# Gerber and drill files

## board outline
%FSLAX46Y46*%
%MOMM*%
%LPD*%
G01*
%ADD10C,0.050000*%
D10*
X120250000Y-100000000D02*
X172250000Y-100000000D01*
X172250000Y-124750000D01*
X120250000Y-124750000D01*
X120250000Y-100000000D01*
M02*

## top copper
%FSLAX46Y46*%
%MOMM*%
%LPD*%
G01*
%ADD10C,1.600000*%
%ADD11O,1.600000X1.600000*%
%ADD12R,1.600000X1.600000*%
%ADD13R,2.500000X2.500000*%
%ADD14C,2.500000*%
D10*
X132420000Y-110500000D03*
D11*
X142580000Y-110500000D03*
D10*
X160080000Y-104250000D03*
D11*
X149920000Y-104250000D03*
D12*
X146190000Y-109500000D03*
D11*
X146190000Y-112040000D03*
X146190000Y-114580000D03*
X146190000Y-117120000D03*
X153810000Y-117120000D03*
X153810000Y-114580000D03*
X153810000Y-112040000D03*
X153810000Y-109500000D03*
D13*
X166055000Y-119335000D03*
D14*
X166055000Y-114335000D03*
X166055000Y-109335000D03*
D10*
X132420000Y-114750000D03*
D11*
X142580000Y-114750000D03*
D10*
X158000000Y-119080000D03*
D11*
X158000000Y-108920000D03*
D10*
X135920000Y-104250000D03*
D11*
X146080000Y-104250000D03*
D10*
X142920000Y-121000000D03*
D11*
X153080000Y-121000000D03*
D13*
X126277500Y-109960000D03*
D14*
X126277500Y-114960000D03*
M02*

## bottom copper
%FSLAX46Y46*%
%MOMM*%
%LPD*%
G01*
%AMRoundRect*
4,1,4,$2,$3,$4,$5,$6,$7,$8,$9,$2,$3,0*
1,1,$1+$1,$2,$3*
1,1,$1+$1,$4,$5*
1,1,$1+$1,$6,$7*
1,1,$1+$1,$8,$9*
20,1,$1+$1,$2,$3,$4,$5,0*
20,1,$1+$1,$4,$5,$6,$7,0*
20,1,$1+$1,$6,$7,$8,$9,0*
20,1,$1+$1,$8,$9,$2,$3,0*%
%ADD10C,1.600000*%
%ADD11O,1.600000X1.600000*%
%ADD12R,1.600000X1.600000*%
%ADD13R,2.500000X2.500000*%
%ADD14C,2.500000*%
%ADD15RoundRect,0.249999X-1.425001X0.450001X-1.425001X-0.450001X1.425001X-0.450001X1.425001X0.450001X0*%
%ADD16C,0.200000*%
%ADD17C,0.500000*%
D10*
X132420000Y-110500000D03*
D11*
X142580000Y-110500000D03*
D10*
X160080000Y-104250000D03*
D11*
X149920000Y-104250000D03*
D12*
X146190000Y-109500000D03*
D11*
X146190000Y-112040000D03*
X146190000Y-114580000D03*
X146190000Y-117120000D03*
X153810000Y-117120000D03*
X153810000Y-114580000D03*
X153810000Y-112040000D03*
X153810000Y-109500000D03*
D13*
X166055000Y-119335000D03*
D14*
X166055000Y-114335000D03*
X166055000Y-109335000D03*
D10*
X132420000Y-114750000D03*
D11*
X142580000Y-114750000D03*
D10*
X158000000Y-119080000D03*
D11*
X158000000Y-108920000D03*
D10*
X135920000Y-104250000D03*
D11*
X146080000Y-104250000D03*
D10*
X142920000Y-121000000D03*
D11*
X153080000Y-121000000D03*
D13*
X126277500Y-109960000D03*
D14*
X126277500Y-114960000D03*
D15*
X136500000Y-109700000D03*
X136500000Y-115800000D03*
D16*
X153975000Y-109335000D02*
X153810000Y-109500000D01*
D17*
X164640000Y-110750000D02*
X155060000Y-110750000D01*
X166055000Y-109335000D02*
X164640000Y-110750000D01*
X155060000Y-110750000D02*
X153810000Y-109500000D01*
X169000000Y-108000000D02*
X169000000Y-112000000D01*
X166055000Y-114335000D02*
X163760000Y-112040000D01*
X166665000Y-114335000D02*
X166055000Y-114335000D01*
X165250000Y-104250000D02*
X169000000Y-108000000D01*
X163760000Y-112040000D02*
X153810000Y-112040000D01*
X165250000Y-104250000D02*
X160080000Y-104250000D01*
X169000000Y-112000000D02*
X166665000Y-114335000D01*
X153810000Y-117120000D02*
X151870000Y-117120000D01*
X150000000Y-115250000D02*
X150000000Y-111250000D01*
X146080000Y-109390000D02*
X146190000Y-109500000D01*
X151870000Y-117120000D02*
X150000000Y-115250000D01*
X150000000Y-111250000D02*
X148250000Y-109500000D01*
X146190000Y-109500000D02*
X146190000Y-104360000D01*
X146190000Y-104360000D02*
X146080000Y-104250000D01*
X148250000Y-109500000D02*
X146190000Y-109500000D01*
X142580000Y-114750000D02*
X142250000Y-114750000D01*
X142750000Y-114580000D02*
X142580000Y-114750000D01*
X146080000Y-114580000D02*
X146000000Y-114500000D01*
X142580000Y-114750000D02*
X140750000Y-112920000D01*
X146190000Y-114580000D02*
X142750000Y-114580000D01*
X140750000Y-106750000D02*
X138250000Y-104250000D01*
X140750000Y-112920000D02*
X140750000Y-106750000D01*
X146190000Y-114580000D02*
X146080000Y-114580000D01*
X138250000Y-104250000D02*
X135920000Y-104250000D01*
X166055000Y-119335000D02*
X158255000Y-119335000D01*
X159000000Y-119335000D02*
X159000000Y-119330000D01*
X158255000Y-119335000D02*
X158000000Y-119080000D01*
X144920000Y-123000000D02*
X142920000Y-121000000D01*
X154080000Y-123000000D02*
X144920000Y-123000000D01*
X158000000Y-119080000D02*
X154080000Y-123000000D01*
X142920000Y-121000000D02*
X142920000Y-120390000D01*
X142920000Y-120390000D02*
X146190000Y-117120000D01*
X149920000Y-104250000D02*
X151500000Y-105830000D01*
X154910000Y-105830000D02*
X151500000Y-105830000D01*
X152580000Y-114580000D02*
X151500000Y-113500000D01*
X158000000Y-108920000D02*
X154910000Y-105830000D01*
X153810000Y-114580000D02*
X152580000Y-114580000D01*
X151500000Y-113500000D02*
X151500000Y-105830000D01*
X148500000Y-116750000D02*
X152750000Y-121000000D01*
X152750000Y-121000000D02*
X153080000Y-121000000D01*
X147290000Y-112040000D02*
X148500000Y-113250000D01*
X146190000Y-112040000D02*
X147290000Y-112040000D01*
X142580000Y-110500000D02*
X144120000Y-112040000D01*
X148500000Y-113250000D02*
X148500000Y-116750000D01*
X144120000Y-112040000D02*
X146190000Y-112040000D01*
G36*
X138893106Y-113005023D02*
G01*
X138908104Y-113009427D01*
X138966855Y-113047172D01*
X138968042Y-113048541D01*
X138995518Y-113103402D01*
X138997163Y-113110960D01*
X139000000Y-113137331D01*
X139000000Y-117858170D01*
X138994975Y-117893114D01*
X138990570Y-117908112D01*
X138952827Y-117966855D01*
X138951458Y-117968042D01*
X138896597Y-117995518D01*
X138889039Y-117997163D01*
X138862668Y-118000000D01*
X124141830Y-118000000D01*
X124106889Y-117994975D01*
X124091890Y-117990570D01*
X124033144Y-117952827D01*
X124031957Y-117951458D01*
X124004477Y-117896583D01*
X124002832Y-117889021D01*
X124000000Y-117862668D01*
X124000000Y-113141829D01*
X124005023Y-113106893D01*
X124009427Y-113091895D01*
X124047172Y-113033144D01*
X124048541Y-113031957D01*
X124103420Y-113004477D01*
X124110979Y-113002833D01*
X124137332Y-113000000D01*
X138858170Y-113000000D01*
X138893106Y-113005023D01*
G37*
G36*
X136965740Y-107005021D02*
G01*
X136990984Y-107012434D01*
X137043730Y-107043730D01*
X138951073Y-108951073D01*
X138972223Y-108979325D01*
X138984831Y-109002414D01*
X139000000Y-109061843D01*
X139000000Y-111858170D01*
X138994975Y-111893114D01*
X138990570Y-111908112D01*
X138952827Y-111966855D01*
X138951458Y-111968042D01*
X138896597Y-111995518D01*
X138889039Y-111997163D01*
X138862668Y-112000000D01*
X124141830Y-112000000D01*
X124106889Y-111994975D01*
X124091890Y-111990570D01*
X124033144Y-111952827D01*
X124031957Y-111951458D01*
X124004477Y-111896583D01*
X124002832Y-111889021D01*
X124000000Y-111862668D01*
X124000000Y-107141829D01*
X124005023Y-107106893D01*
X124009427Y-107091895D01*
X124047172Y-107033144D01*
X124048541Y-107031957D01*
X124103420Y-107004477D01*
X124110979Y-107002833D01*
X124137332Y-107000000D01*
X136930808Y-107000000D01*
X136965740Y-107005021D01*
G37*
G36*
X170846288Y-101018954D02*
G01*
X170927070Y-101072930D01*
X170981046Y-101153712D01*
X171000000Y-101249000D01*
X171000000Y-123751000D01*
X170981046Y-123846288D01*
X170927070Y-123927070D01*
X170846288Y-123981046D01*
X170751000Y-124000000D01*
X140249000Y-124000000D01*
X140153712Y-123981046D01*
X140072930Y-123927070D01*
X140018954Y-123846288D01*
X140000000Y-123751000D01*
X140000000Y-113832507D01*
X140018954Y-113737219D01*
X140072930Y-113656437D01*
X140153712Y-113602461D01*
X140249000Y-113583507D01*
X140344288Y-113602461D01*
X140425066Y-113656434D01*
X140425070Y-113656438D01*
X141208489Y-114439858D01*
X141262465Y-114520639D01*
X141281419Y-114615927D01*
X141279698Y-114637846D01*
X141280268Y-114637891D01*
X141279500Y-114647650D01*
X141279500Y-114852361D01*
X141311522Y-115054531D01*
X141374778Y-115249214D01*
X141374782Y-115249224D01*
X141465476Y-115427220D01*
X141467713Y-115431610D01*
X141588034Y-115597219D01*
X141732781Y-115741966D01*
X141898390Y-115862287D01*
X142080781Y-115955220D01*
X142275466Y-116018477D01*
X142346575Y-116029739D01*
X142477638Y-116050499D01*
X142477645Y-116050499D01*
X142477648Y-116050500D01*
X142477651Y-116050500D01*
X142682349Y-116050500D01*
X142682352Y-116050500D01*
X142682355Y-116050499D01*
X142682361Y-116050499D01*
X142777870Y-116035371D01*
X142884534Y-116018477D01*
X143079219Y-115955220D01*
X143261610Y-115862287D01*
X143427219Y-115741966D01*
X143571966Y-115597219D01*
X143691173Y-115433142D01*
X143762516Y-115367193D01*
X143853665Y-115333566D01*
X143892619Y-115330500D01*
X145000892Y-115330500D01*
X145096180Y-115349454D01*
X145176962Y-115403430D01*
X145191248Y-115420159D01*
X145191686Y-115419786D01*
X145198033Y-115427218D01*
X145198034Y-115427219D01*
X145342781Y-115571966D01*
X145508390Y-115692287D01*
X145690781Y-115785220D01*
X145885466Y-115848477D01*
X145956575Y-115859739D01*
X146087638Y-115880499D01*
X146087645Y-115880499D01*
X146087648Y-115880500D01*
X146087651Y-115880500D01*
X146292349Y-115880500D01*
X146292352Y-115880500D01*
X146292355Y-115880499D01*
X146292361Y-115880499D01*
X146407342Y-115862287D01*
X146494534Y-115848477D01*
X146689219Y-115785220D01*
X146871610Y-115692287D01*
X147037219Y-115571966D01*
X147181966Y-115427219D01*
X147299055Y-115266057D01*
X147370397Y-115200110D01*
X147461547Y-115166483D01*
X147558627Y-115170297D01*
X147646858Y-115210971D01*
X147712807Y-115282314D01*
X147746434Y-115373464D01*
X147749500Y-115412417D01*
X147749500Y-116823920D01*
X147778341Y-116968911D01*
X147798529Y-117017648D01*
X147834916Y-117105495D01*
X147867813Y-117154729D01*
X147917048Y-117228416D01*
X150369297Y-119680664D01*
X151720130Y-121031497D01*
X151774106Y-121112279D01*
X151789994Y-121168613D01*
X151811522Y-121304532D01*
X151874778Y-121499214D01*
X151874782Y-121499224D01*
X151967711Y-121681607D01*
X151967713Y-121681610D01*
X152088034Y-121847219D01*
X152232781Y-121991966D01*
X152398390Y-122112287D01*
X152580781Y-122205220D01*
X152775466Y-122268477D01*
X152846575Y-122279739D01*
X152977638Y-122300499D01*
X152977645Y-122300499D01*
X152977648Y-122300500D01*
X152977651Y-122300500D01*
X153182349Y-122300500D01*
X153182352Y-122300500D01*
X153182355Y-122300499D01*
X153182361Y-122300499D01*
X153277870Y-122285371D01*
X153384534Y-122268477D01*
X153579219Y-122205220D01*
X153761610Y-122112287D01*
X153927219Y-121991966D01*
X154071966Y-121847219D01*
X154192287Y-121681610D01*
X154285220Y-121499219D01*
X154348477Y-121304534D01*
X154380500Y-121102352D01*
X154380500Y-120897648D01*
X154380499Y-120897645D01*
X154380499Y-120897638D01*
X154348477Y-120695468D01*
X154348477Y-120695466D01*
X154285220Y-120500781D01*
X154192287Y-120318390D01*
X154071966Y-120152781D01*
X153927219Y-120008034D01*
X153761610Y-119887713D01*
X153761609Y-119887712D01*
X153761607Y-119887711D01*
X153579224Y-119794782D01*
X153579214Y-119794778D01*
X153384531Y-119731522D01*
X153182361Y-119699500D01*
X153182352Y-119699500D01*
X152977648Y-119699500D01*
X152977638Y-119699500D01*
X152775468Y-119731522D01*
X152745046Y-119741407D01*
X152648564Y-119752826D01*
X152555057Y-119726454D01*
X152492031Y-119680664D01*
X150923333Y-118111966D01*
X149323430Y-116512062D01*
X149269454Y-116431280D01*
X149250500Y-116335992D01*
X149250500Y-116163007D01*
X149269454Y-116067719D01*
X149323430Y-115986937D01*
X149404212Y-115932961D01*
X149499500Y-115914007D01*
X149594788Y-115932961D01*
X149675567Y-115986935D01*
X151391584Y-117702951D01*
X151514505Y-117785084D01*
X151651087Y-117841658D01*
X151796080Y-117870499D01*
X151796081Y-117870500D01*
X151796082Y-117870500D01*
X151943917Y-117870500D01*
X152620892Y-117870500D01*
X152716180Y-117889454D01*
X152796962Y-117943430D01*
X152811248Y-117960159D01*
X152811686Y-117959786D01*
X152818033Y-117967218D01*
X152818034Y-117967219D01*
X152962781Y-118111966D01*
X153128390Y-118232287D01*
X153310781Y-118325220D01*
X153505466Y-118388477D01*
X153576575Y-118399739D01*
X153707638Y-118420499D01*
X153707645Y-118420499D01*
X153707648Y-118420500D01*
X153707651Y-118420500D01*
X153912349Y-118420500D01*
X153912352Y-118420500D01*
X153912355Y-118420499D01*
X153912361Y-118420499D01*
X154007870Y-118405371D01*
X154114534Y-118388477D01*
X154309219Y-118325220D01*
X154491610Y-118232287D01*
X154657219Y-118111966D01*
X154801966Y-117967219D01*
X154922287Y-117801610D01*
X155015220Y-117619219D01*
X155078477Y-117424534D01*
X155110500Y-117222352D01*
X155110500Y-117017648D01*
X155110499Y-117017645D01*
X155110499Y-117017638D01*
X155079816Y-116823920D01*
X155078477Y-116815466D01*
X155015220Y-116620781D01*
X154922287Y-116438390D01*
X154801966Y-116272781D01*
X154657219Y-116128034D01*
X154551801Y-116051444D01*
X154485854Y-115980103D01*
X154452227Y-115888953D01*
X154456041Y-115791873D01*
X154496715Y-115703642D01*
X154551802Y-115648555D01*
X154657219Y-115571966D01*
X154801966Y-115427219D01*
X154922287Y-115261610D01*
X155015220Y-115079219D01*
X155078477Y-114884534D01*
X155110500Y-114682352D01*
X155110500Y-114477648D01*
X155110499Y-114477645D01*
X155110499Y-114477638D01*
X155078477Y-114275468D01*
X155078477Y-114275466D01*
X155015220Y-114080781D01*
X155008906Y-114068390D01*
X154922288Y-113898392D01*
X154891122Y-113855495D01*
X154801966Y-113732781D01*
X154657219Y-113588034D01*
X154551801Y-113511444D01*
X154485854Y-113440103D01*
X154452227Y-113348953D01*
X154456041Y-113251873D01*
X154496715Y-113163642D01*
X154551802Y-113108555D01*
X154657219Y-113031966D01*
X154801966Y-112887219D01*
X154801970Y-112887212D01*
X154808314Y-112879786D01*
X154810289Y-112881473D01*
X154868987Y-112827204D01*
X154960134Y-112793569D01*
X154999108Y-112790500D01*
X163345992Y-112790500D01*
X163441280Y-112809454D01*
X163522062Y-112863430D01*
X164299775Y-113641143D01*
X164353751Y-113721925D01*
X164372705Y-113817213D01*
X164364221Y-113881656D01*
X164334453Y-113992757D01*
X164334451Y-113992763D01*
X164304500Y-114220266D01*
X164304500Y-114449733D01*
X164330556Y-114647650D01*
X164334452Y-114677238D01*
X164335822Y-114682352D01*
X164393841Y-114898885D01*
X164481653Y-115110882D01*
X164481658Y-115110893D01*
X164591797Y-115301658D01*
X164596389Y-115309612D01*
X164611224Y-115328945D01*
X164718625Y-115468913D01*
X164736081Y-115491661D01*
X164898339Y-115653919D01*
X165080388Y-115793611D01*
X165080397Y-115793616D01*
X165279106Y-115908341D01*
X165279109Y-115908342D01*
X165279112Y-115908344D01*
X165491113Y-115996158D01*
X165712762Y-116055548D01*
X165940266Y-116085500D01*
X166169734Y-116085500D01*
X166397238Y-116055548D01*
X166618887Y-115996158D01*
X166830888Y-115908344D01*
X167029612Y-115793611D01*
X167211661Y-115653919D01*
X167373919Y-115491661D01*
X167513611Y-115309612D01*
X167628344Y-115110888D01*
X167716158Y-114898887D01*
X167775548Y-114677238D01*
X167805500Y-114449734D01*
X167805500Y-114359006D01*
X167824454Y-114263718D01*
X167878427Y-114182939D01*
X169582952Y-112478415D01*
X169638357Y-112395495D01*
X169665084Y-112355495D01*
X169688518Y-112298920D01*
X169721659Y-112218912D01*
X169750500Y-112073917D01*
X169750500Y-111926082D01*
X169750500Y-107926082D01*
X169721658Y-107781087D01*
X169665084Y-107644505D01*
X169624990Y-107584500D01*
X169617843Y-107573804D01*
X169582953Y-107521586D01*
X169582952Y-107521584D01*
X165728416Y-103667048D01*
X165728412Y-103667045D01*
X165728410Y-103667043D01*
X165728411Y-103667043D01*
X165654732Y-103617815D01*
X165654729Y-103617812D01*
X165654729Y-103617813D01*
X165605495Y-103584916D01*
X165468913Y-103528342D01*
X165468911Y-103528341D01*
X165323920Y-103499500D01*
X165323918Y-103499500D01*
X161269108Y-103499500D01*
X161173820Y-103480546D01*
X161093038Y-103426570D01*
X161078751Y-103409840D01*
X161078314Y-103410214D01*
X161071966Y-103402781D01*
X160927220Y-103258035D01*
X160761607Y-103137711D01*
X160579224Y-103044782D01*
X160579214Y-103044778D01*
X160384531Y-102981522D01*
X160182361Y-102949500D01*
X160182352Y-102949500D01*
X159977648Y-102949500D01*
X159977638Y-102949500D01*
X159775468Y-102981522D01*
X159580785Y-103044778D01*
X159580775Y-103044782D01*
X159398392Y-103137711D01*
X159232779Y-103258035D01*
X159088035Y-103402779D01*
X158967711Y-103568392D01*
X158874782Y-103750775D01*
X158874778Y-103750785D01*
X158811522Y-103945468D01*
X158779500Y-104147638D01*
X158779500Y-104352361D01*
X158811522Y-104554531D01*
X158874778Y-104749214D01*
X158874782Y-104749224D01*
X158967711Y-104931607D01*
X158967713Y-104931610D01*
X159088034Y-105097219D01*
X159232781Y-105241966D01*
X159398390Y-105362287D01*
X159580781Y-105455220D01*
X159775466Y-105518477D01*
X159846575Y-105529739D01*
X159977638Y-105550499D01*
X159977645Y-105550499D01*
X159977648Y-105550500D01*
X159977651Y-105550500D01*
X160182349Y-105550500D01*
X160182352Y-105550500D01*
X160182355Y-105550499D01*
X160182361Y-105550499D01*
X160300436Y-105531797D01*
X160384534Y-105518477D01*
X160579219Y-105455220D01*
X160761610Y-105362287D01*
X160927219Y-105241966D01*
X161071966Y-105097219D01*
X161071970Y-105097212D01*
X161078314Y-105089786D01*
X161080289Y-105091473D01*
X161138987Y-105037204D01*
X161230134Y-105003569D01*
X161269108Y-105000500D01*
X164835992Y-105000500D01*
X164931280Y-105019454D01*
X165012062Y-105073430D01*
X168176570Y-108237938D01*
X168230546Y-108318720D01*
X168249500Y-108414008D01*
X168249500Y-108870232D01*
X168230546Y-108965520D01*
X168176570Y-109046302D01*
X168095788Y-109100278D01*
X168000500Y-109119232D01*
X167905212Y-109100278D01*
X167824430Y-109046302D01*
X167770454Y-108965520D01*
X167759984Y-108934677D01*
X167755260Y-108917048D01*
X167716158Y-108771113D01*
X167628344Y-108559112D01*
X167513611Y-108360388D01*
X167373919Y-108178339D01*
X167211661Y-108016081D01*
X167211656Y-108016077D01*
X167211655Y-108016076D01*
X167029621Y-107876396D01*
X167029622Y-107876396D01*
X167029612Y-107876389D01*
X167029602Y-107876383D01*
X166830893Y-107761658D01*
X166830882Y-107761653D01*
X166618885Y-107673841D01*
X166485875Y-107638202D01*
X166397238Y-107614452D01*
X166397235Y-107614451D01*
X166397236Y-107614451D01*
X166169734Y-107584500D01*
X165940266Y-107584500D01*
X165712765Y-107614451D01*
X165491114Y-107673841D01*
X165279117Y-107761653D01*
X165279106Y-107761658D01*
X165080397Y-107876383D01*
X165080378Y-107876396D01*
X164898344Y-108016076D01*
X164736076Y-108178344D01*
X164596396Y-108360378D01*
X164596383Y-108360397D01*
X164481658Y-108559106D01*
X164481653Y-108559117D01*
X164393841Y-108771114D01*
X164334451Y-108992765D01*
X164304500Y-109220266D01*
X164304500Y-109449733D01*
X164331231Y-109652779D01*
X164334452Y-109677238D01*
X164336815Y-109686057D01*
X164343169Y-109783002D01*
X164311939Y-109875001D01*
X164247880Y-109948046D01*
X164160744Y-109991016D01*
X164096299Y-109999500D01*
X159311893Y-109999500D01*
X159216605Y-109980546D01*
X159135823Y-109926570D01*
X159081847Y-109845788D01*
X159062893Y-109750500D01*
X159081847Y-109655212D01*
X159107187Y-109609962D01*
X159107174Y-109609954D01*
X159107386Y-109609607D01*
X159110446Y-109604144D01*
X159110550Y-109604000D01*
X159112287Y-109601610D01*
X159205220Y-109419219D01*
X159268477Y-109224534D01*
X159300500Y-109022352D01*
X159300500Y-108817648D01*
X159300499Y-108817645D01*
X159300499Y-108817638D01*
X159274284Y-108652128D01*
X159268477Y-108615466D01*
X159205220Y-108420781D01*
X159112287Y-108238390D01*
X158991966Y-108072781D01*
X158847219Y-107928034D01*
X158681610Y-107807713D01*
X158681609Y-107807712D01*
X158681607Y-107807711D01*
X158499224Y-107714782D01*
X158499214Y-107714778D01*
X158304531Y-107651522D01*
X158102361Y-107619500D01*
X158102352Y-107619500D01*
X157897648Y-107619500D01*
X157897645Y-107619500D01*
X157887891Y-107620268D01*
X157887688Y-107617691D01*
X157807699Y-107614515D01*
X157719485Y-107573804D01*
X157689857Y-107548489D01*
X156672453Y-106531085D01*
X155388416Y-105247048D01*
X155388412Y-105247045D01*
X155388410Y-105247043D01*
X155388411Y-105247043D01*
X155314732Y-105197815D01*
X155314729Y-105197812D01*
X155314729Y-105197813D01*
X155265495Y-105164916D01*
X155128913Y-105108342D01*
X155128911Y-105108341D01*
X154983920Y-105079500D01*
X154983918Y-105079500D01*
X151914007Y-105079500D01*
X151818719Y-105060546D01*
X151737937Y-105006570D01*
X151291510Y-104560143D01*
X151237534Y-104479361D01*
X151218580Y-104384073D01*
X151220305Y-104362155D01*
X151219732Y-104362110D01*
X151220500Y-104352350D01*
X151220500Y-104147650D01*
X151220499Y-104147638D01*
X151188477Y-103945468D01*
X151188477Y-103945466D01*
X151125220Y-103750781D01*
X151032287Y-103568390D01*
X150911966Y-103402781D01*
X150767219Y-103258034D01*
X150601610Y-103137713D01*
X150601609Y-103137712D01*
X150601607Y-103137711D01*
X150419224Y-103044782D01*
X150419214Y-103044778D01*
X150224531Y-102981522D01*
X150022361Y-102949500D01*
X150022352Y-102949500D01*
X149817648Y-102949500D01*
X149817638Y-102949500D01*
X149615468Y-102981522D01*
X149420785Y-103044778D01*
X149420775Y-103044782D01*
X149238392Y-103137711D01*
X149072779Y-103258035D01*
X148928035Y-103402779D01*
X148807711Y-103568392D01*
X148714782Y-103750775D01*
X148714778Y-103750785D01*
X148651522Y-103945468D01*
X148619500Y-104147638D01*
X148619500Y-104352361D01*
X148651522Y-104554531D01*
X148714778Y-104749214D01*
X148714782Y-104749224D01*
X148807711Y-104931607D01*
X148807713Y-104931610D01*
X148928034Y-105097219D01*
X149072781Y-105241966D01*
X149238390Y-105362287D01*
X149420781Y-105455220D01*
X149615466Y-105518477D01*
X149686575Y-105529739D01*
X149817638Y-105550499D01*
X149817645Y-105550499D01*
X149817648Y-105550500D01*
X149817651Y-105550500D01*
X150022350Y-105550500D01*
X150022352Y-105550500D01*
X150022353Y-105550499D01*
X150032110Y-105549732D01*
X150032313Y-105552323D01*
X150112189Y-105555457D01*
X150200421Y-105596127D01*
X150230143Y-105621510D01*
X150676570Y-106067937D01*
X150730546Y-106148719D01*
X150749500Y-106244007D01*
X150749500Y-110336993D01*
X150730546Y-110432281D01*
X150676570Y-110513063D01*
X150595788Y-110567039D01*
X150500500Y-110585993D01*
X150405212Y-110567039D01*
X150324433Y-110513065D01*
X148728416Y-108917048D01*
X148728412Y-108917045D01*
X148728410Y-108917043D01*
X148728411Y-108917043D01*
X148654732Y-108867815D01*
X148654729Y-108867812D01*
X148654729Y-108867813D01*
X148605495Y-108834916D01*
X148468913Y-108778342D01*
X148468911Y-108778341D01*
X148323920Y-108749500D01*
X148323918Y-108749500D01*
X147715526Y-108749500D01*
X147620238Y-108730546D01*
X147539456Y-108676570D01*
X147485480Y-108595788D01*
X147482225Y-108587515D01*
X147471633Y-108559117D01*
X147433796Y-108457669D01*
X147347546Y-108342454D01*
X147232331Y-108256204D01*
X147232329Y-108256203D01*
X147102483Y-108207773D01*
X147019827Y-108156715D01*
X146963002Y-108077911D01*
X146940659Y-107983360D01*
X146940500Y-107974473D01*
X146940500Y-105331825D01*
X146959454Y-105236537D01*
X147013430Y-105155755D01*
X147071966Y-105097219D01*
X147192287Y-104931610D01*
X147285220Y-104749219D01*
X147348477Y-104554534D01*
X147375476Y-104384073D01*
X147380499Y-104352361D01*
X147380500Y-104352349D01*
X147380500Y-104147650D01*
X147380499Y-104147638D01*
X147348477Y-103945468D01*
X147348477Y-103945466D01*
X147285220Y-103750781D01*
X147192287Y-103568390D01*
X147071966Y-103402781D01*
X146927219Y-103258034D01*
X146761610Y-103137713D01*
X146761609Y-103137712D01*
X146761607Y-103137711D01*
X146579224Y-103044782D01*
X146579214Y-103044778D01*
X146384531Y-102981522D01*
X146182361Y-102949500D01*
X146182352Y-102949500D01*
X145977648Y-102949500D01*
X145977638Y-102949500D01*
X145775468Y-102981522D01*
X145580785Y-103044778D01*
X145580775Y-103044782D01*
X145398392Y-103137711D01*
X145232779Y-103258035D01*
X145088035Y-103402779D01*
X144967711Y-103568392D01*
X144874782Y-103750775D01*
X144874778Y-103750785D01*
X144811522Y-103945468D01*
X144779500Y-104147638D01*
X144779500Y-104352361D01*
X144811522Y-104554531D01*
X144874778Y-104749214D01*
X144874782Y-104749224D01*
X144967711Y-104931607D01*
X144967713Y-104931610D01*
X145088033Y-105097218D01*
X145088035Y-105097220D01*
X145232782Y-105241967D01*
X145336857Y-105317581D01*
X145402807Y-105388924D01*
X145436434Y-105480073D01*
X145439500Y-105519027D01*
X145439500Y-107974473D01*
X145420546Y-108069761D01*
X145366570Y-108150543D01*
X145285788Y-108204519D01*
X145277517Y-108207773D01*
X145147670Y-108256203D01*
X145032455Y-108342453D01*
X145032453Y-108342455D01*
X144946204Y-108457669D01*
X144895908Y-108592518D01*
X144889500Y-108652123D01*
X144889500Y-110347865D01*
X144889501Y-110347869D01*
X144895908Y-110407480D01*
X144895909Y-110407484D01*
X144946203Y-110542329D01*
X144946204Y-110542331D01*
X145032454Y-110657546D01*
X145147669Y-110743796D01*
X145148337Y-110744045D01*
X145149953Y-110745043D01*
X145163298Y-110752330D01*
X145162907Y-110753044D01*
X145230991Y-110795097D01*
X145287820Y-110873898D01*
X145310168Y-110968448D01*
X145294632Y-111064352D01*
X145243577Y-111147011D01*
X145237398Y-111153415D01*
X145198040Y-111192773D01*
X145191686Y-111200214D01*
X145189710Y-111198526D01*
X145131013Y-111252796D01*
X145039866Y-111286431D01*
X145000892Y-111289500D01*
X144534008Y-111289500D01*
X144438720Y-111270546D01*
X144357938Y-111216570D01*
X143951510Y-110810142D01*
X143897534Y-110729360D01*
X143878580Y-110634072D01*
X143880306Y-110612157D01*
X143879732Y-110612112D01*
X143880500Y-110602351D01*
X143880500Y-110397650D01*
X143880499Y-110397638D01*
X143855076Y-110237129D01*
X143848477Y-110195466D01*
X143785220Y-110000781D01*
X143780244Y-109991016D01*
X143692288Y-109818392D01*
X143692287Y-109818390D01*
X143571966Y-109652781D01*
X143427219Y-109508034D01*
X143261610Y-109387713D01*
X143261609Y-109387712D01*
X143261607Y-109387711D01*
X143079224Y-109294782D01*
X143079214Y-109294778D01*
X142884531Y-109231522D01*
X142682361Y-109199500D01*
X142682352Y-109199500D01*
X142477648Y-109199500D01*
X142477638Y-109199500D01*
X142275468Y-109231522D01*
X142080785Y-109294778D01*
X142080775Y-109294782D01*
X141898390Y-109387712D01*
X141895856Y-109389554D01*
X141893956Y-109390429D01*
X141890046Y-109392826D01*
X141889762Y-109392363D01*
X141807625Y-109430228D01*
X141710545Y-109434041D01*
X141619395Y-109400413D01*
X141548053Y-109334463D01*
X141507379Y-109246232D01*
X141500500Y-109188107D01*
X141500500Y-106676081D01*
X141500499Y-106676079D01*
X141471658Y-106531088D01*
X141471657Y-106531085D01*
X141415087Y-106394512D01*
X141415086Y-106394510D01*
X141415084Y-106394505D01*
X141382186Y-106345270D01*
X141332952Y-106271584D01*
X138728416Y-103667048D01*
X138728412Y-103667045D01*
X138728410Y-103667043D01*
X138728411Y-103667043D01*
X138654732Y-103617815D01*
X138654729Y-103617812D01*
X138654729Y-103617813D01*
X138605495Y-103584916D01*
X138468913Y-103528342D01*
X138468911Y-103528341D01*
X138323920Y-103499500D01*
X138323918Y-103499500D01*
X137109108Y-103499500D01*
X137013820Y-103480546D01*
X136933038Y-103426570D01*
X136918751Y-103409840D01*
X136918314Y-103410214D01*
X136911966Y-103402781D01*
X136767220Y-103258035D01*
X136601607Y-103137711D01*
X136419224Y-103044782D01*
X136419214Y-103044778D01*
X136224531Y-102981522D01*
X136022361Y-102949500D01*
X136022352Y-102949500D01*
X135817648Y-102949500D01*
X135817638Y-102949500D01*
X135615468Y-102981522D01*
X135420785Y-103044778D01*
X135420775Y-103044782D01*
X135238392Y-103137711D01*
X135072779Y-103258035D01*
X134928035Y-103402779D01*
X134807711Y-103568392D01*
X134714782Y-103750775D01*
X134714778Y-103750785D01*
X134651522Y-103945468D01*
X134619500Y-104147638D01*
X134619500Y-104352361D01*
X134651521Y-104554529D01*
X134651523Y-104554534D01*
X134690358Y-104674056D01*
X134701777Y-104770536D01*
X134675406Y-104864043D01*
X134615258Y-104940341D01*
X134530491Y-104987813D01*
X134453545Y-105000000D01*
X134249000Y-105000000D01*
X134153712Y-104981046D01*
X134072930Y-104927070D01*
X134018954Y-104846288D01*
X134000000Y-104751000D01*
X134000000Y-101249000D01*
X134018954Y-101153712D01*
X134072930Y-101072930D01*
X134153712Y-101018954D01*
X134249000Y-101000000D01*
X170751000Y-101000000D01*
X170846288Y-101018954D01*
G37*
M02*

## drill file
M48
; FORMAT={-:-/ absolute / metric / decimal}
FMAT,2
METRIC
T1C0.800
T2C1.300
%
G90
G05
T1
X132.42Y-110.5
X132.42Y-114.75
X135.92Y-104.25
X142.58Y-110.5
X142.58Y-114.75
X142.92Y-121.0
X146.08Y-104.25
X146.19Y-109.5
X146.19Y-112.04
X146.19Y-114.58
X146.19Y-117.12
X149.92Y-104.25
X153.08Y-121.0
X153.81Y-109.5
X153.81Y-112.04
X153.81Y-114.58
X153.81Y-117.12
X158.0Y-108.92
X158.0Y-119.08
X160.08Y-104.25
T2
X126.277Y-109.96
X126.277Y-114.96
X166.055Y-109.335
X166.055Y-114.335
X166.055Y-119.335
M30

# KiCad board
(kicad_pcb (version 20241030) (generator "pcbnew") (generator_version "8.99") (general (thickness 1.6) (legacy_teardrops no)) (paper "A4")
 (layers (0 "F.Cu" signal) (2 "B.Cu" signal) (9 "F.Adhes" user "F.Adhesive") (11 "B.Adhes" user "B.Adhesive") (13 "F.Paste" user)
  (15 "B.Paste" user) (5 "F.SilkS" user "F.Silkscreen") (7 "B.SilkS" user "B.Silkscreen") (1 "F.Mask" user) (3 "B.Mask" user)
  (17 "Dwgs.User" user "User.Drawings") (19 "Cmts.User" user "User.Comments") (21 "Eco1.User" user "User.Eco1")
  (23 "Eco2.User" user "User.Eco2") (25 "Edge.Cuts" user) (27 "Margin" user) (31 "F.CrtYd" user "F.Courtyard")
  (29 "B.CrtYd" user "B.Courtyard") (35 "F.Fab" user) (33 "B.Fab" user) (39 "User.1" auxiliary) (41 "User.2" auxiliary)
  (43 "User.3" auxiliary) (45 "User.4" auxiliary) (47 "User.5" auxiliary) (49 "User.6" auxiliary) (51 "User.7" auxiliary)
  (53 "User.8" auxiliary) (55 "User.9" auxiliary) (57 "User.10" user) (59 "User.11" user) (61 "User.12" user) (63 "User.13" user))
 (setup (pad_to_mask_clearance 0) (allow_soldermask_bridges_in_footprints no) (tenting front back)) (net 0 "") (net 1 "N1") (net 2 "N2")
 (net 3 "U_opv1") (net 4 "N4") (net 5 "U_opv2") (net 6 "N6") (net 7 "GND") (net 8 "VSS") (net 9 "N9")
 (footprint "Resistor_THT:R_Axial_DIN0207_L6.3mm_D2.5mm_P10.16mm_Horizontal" (layer "F.Cu") (at 132.42 110.5)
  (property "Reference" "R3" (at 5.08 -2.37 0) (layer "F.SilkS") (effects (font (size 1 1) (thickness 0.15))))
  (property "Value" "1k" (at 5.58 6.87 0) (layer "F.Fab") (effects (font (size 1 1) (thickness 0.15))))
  (pad "1" thru_hole circle (at 0 0) (size 1.6 1.6) (drill 0.8) (layers "*.Cu" "*.Mask") (remove_unused_layers no) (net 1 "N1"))
  (pad "2" thru_hole oval (at 10.16 0) (size 1.6 1.6) (drill 0.8) (layers "*.Cu" "*.Mask") (remove_unused_layers no) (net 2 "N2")))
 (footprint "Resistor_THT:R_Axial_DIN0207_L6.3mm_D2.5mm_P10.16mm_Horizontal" (layer "F.Cu") (at 160.08 104.25 180)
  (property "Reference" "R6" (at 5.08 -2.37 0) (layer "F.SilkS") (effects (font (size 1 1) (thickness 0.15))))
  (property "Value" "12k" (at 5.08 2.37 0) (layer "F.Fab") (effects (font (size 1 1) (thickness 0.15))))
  (pad "1" thru_hole circle (at 0 0 180) (size 1.6 1.6) (drill 0.8) (layers "*.Cu" "*.Mask") (remove_unused_layers no) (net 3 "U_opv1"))
  (pad "2" thru_hole oval (at 10.16 0 180) (size 1.6 1.6) (drill 0.8) (layers "*.Cu" "*.Mask") (remove_unused_layers no) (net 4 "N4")))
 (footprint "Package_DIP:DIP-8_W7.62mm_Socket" (layer "F.Cu") (at 146.19 109.5)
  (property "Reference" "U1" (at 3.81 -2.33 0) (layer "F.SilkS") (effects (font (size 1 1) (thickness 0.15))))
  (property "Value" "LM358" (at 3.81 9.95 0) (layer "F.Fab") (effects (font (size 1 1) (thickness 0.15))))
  (pad "1" thru_hole rect (at 0 0) (size 1.6 1.6) (drill 0.8) (layers "*.Cu" "*.Mask") (remove_unused_layers no) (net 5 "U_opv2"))
  (pad "2" thru_hole oval (at 0 2.54) (size 1.6 1.6) (drill 0.8) (layers "*.Cu" "*.Mask") (remove_unused_layers no) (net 2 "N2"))
  (pad "3" thru_hole oval (at 0 5.08) (size 1.6 1.6) (drill 0.8) (layers "*.Cu" "*.Mask") (remove_unused_layers no) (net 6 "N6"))
  (pad "4" thru_hole oval (at 0 7.62) (size 1.6 1.6) (drill 0.8) (layers "*.Cu" "*.Mask") (remove_unused_layers no) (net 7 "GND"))
  (pad "5" thru_hole oval (at 7.62 7.62) (size 1.6 1.6) (drill 0.8) (layers "*.Cu" "*.Mask") (remove_unused_layers no) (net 5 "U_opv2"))
  (pad "6" thru_hole oval (at 7.62 5.08) (size 1.6 1.6) (drill 0.8) (layers "*.Cu" "*.Mask") (remove_unused_layers no) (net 4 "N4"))
  (pad "7" thru_hole oval (at 7.62 2.54) (size 1.6 1.6) (drill 0.8) (layers "*.Cu" "*.Mask") (remove_unused_layers no) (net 3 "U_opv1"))
  (pad "8" thru_hole oval (at 7.62 0) (size 1.6 1.6) (drill 0.8) (layers "*.Cu" "*.Mask") (remove_unused_layers no) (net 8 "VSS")))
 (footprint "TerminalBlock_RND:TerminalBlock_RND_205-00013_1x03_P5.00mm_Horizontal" (layer "F.Cu") (at 166.055 119.335 90)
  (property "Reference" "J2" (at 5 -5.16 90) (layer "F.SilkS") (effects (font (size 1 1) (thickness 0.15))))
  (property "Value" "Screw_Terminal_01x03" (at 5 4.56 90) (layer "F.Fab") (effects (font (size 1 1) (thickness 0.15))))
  (pad "1" thru_hole rect (at 0 0 90) (size 2.5 2.5) (drill 1.3) (layers "*.Cu" "*.Mask") (remove_unused_layers no) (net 7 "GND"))
  (pad "2" thru_hole circle (at 5 0 90) (size 2.5 2.5) (drill 1.3) (layers "*.Cu" "*.Mask") (remove_unused_layers no) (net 3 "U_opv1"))
  (pad "3" thru_hole circle (at 10 0 90) (size 2.5 2.5) (drill 1.3) (layers "*.Cu" "*.Mask") (remove_unused_layers no) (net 8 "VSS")))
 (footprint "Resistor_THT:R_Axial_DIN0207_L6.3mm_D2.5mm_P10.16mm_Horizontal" (layer "F.Cu") (at 132.42 114.75)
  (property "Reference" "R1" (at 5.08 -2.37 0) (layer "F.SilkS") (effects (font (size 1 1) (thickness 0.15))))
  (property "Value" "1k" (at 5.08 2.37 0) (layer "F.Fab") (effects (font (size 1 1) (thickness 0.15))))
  (pad "1" thru_hole circle (at 0 0) (size 1.6 1.6) (drill 0.8) (layers "*.Cu" "*.Mask") (remove_unused_layers no) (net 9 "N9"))
  (pad "2" thru_hole oval (at 10.16 0) (size 1.6 1.6) (drill 0.8) (layers "*.Cu" "*.Mask") (remove_unused_layers no) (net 6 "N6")))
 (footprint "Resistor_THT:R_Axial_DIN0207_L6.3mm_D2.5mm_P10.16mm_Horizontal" (layer "F.Cu") (at 158 119.08 90)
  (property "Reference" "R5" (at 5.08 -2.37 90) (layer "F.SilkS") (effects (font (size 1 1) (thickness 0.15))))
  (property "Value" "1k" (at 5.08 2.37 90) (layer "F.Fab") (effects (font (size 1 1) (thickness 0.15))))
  (pad "1" thru_hole circle (at 0 0 90) (size 1.6 1.6) (drill 0.8) (layers "*.Cu" "*.Mask") (remove_unused_layers no) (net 7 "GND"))
  (pad "2" thru_hole oval (at 10.16 0 90) (size 1.6 1.6) (drill 0.8) (layers "*.Cu" "*.Mask") (remove_unused_layers no) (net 4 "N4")))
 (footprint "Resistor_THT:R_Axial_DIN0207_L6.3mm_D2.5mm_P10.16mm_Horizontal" (layer "F.Cu") (at 135.92 104.25)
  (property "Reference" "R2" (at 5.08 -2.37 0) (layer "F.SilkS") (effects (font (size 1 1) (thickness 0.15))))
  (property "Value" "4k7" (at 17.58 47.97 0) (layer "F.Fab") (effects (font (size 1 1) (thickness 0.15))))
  (pad "1" thru_hole circle (at 0 0) (size 1.6 1.6) (drill 0.8) (layers "*.Cu" "*.Mask") (remove_unused_layers no) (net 6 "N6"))
  (pad "2" thru_hole oval (at 10.16 0) (size 1.6 1.6) (drill 0.8) (layers "*.Cu" "*.Mask") (remove_unused_layers no) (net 5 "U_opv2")))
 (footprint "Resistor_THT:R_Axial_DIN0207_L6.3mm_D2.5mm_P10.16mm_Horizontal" (layer "F.Cu") (at 142.92 121)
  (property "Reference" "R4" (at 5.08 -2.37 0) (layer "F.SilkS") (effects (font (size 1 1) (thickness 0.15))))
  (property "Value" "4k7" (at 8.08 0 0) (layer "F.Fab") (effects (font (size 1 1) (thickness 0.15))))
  (pad "1" thru_hole circle (at 0 0) (size 1.6 1.6) (drill 0.8) (layers "*.Cu" "*.Mask") (remove_unused_layers no) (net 7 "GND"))
  (pad "2" thru_hole oval (at 10.16 0) (size 1.6 1.6) (drill 0.8) (layers "*.Cu" "*.Mask") (remove_unused_layers no) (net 2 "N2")))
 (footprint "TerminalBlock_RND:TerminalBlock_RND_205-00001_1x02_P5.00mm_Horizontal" (layer "F.Cu") (at 126.2775 109.96 -90)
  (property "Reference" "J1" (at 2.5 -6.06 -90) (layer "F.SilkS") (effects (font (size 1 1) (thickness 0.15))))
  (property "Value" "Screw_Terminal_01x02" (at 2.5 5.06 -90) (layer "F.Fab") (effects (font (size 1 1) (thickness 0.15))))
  (pad "1" thru_hole rect (at 0 0 270) (size 2.5 2.5) (drill 1.3) (layers "*.Cu" "*.Mask") (remove_unused_layers no) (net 1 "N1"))
  (pad "2" thru_hole circle (at 5 0 270) (size 2.5 2.5) (drill 1.3) (layers "*.Cu" "*.Mask") (remove_unused_layers no) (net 9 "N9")))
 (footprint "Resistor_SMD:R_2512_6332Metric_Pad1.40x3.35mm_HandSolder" (layer "B.Cu") (at 136.5 112.75 -90)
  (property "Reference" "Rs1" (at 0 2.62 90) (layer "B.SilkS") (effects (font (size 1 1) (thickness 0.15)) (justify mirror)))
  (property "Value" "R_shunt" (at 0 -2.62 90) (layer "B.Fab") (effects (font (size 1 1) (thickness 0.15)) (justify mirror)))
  (pad "1" smd roundrect (at -3.05 0 270) (size 1.4 3.35) (layers "B.Cu" "B.Mask" "B.Paste") (roundrect_rratio 0.178571) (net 1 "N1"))
  (pad "2" smd roundrect (at 3.05 0 270) (size 1.4 3.35) (layers "B.Cu" "B.Mask" "B.Paste") (roundrect_rratio 0.178571) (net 9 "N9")))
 (gr_rect (start 120.25 100) (end 172.25 124.75) (stroke (width 0.05) (type default)) (fill none) (layer "Edge.Cuts"))
 (segment (start 153.975 109.335) (end 153.81 109.5) (width 0.2) (layer "B.Cu") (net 8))
 (segment (start 164.64 110.75) (end 155.06 110.75) (width 0.5) (layer "B.Cu") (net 8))
 (segment (start 166.055 109.335) (end 164.64 110.75) (width 0.5) (layer "B.Cu") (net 8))
 (segment (start 155.06 110.75) (end 153.81 109.5) (width 0.5) (layer "B.Cu") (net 8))
 (segment (start 169 108) (end 169 112) (width 0.5) (layer "B.Cu") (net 3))
 (segment (start 166.055 114.335) (end 163.76 112.04) (width 0.5) (layer "B.Cu") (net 3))
 (segment (start 166.665 114.335) (end 166.055 114.335) (width 0.5) (layer "B.Cu") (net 3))
 (segment (start 165.25 104.25) (end 169 108) (width 0.5) (layer "B.Cu") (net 3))
 (segment (start 163.76 112.04) (end 153.81 112.04) (width 0.5) (layer "B.Cu") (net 3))
 (segment (start 165.25 104.25) (end 160.08 104.25) (width 0.5) (layer "B.Cu") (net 3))
 (segment (start 169 112) (end 166.665 114.335) (width 0.5) (layer "B.Cu") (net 3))
 (segment (start 153.81 117.12) (end 151.87 117.12) (width 0.5) (layer "B.Cu") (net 5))
 (segment (start 150 115.25) (end 150 111.25) (width 0.5) (layer "B.Cu") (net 5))
 (segment (start 146.08 109.39) (end 146.19 109.5) (width 0.5) (layer "B.Cu") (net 5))
 (segment (start 151.87 117.12) (end 150 115.25) (width 0.5) (layer "B.Cu") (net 5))
 (segment (start 150 111.25) (end 148.25 109.5) (width 0.5) (layer "B.Cu") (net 5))
 (segment (start 146.19 109.5) (end 146.19 104.36) (width 0.5) (layer "B.Cu") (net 5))
 (segment (start 146.19 104.36) (end 146.08 104.25) (width 0.5) (layer "B.Cu") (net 5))
 (segment (start 148.25 109.5) (end 146.19 109.5) (width 0.5) (layer "B.Cu") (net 5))
 (segment (start 142.58 114.75) (end 142.25 114.75) (width 0.5) (layer "B.Cu") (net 6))
 (segment (start 142.75 114.58) (end 142.58 114.75) (width 0.5) (layer "B.Cu") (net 6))
 (segment (start 146.08 114.58) (end 146 114.5) (width 0.5) (layer "B.Cu") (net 6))
 (segment (start 142.58 114.75) (end 140.75 112.92) (width 0.5) (layer "B.Cu") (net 6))
 (segment (start 146.19 114.58) (end 142.75 114.58) (width 0.5) (layer "B.Cu") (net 6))
 (segment (start 140.75 106.75) (end 138.25 104.25) (width 0.5) (layer "B.Cu") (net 6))
 (segment (start 140.75 112.92) (end 140.75 106.75) (width 0.5) (layer "B.Cu") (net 6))
 (segment (start 146.19 114.58) (end 146.08 114.58) (width 0.5) (layer "B.Cu") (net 6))
 (segment (start 138.25 104.25) (end 135.92 104.25) (width 0.5) (layer "B.Cu") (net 6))
 (segment (start 166.055 119.335) (end 158.255 119.335) (width 0.5) (layer "B.Cu") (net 7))
 (segment (start 159 119.335) (end 159 119.33) (width 0.5) (layer "B.Cu") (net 7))
 (segment (start 158.255 119.335) (end 158 119.08) (width 0.5) (layer "B.Cu") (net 7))
 (segment (start 144.92 123) (end 142.92 121) (width 0.5) (layer "B.Cu") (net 7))
 (segment (start 154.08 123) (end 144.92 123) (width 0.5) (layer "B.Cu") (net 7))
 (segment (start 158 119.08) (end 154.08 123) (width 0.5) (layer "B.Cu") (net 7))
 (segment (start 142.92 121) (end 142.92 120.39) (width 0.5) (layer "B.Cu") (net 7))
 (segment (start 142.92 120.39) (end 146.19 117.12) (width 0.5) (layer "B.Cu") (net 7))
 (segment (start 149.92 104.25) (end 151.5 105.83) (width 0.5) (layer "B.Cu") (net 4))
 (segment (start 154.91 105.83) (end 151.5 105.83) (width 0.5) (layer "B.Cu") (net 4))
 (segment (start 152.58 114.58) (end 151.5 113.5) (width 0.5) (layer "B.Cu") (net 4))
 (segment (start 158 108.92) (end 154.91 105.83) (width 0.5) (layer "B.Cu") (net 4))
 (segment (start 153.81 114.58) (end 152.58 114.58) (width 0.5) (layer "B.Cu") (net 4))
 (segment (start 151.5 113.5) (end 151.5 105.83) (width 0.5) (layer "B.Cu") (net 4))
 (segment (start 148.5 116.75) (end 152.75 121) (width 0.5) (layer "B.Cu") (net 2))
 (segment (start 152.75 121) (end 153.08 121) (width 0.5) (layer "B.Cu") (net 2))
 (segment (start 147.29 112.04) (end 148.5 113.25) (width 0.5) (layer "B.Cu") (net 2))
 (segment (start 146.19 112.04) (end 147.29 112.04) (width 0.5) (layer "B.Cu") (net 2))
 (segment (start 142.58 110.5) (end 144.12 112.04) (width 0.5) (layer "B.Cu") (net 2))
 (segment (start 148.5 113.25) (end 148.5 116.75) (width 0.5) (layer "B.Cu") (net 2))
 (segment (start 144.12 112.04) (end 146.19 112.04) (width 0.5) (layer "B.Cu") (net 2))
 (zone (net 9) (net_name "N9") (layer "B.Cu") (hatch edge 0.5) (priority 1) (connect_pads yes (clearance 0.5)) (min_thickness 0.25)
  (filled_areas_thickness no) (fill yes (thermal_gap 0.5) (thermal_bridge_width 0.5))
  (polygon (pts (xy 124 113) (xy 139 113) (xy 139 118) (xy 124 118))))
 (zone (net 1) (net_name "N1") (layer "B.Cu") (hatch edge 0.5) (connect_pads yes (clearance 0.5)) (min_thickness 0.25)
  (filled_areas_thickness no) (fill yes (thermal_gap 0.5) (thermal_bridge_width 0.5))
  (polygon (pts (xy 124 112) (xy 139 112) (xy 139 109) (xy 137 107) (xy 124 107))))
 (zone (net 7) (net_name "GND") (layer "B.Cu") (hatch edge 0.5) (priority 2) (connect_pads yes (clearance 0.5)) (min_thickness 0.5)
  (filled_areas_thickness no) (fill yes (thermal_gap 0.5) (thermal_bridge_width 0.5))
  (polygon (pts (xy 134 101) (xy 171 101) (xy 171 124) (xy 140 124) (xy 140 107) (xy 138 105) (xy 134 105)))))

